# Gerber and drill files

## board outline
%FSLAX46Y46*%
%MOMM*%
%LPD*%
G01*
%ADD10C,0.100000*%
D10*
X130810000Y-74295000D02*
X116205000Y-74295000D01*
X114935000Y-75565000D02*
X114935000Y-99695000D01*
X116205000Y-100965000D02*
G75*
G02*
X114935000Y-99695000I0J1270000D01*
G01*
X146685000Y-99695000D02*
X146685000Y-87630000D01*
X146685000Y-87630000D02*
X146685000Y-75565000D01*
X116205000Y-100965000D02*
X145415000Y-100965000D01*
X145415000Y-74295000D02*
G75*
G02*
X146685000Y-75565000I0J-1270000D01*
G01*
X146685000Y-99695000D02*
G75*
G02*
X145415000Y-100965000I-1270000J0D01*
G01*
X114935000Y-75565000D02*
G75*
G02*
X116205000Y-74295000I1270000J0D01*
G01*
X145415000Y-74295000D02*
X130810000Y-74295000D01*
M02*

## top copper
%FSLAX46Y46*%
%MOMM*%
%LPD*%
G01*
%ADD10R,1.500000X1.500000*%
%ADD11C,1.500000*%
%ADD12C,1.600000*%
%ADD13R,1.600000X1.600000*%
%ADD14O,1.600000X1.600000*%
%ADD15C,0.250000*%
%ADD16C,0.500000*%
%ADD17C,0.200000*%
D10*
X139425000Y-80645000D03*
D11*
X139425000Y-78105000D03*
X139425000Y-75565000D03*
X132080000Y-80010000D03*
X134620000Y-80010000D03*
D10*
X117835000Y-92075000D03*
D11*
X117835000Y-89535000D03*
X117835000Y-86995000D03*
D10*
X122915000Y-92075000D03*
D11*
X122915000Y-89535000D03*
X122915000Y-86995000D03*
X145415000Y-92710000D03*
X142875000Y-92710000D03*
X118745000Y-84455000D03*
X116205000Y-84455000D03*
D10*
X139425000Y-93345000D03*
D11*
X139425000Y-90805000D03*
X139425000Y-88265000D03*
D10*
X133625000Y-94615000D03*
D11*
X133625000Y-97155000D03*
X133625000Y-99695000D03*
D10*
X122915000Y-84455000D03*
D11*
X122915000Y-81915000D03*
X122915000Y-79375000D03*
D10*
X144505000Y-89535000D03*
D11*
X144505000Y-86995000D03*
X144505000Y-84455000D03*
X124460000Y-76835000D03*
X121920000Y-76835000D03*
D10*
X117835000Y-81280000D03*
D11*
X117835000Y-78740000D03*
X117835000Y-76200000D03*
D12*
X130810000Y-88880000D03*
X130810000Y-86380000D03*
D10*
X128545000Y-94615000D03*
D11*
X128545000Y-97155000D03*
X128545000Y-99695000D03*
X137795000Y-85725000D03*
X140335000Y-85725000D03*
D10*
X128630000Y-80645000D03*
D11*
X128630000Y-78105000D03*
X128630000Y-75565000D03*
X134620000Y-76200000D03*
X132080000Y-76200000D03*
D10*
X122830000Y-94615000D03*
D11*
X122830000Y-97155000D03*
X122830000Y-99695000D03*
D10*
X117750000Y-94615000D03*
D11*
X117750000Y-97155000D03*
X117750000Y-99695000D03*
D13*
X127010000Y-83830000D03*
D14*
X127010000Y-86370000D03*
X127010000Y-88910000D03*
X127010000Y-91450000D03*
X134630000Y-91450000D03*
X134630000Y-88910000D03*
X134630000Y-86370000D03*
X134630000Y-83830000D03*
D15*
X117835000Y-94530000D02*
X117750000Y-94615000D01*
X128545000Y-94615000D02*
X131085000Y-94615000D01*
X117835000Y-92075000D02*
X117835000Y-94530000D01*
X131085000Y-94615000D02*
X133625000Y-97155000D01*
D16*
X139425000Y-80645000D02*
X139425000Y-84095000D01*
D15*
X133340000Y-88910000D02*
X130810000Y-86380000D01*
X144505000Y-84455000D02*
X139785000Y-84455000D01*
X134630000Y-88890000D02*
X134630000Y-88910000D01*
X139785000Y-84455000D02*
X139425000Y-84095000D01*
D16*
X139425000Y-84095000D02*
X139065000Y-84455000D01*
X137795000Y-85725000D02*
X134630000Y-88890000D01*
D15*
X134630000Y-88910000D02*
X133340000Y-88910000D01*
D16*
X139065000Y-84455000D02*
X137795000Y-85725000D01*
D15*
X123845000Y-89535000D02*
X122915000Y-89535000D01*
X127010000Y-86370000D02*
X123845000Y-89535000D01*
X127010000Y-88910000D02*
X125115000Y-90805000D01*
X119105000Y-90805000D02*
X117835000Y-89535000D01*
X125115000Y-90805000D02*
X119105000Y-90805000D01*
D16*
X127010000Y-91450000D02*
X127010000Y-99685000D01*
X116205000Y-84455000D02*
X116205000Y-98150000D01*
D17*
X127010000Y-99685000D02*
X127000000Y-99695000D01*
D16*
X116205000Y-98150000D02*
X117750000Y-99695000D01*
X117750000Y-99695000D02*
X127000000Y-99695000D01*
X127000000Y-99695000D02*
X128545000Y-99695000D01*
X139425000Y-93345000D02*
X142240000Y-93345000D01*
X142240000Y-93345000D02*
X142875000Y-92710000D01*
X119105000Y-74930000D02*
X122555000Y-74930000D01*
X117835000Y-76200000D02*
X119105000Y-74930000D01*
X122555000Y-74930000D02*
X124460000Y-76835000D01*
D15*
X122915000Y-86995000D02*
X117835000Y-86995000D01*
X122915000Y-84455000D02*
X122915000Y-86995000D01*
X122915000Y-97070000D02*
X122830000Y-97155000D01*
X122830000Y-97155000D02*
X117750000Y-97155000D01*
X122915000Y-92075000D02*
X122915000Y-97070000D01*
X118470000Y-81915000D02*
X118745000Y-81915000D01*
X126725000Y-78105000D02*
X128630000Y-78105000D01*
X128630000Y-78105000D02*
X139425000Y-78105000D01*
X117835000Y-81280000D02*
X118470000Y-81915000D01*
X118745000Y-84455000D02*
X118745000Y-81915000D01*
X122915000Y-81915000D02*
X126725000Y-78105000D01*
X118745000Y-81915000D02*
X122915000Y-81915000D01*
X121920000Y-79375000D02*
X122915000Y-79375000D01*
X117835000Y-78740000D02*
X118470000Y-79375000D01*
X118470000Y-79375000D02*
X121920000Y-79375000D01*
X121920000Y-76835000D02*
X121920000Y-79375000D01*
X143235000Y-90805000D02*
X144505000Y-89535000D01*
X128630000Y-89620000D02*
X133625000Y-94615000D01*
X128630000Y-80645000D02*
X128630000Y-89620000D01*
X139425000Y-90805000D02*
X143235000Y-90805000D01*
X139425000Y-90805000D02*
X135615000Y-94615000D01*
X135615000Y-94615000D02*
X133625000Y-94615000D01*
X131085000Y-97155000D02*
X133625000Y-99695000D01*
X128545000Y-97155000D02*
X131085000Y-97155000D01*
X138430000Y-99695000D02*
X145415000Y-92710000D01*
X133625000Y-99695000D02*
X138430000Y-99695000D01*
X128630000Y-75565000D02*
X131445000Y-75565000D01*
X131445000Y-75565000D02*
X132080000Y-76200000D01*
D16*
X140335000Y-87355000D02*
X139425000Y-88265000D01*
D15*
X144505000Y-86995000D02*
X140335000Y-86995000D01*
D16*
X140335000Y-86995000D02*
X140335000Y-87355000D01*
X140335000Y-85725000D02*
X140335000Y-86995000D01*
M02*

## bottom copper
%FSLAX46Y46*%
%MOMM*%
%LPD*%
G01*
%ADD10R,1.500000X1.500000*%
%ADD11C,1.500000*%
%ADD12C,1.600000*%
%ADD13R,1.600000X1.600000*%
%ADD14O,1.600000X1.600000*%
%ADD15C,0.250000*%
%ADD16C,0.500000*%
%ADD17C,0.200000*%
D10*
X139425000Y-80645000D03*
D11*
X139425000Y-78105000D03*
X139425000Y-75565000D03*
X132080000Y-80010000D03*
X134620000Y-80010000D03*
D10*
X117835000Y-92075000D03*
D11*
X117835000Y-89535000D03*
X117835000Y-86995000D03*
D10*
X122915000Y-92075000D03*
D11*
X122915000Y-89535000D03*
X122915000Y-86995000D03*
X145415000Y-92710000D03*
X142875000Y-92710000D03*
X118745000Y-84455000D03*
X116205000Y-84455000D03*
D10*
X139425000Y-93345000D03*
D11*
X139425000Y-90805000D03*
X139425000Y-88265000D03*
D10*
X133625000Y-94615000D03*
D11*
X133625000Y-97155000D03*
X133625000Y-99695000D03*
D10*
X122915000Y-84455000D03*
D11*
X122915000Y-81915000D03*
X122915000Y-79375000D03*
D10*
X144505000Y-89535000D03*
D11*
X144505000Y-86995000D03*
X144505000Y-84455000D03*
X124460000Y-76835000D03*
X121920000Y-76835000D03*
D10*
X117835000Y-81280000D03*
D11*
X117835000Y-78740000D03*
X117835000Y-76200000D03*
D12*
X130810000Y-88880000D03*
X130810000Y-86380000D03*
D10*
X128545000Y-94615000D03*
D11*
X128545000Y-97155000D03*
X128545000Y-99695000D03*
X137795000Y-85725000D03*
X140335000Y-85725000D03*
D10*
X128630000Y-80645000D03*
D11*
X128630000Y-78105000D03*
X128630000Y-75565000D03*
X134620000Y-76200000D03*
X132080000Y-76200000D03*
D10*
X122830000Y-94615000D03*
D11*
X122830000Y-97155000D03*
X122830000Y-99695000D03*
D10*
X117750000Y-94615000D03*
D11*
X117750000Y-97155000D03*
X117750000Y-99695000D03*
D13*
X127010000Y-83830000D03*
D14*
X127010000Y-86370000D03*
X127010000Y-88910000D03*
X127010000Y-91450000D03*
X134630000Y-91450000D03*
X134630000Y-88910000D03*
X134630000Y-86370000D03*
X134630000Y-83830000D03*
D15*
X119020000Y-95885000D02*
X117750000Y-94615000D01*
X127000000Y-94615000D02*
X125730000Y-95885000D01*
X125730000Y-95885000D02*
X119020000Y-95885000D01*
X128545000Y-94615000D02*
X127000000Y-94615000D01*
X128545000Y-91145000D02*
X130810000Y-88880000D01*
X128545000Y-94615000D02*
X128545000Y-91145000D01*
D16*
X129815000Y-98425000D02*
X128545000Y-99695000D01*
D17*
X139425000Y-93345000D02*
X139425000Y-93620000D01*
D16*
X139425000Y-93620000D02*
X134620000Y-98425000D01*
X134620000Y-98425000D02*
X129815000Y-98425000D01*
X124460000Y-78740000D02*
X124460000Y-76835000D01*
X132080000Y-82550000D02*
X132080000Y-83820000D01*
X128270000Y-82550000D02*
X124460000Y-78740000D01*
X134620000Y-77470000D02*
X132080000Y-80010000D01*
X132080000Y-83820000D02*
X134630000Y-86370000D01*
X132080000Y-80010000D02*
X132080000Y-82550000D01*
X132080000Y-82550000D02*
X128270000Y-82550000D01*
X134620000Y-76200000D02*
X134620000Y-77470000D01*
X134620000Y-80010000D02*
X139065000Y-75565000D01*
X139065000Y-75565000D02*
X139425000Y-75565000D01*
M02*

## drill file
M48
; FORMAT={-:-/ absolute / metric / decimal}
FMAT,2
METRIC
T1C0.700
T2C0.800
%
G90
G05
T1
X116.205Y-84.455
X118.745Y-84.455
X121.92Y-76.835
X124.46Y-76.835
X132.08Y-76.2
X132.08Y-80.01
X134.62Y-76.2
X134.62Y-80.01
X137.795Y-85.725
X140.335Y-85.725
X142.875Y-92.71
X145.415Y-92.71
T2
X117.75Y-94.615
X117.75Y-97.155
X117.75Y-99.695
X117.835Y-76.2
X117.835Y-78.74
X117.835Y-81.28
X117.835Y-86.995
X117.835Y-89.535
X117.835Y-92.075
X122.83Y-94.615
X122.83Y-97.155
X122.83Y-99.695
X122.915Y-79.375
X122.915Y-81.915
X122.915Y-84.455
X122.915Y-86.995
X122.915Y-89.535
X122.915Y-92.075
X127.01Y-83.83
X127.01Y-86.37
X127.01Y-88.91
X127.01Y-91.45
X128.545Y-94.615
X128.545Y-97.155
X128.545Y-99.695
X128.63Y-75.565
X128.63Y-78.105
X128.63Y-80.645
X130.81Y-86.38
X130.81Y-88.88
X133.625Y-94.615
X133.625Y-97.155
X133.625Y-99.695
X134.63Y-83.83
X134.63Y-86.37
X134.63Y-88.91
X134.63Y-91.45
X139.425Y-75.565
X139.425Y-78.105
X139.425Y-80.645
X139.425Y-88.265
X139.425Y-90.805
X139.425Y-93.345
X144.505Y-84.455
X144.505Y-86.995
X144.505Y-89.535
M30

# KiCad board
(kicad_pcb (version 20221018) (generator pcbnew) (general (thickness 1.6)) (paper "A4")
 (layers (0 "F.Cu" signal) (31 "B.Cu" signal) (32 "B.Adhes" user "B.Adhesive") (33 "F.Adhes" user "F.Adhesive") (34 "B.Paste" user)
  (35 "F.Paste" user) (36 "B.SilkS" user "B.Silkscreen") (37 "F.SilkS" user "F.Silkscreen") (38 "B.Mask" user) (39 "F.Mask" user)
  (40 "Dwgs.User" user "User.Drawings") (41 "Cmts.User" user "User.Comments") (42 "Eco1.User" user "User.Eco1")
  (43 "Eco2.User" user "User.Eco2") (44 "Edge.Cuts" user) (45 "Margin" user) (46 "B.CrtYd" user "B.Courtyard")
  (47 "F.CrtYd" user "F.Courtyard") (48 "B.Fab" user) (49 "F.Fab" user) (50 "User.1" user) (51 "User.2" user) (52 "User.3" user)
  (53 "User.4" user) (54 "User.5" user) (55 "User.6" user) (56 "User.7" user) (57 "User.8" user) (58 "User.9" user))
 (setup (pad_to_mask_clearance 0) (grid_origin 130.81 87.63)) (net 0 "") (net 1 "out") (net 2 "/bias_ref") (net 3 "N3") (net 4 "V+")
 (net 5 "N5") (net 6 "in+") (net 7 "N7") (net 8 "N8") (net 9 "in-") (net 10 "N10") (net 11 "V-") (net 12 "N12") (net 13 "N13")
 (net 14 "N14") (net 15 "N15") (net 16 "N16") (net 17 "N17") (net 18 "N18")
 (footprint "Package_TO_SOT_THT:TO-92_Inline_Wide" (layer "F.Cu") (at 139.425 80.645 90)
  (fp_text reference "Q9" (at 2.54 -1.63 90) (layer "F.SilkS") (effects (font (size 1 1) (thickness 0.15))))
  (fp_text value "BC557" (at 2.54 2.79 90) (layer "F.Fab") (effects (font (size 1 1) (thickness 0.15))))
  (pad "1" thru_hole rect (at 0 0 90) (size 1.5 1.5) (drill 0.8) (layers "*.Cu" "*.Mask") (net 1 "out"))
  (pad "2" thru_hole circle (at 2.54 0 90) (size 1.5 1.5) (drill 0.8) (layers "*.Cu" "*.Mask") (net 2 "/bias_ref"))
  (pad "3" thru_hole circle (at 5.08 0 90) (size 1.5 1.5) (drill 0.8) (layers "*.Cu" "*.Mask") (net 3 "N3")))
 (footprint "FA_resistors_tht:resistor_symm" (layer "F.Cu") (at 133.35 80.01)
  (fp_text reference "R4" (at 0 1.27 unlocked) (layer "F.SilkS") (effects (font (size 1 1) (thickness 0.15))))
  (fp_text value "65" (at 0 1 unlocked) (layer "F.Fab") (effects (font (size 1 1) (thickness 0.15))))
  (pad "1" thru_hole circle (at -1.27 0) (size 1.5 1.5) (drill 0.7) (layers "*.Cu" "*.Mask") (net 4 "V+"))
  (pad "2" thru_hole circle (at 1.27 0) (size 1.5 1.5) (drill 0.7) (layers "*.Cu" "*.Mask") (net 3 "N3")))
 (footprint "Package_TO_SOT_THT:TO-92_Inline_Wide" (layer "F.Cu") (at 117.835 92.075 90)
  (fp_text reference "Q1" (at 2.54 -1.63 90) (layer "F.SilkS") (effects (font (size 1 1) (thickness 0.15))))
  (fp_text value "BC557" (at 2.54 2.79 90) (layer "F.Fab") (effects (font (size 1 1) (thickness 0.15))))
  (pad "1" thru_hole rect (at 0 0 90) (size 1.5 1.5) (drill 0.8) (layers "*.Cu" "*.Mask") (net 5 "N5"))
  (pad "2" thru_hole circle (at 2.54 0 90) (size 1.5 1.5) (drill 0.8) (layers "*.Cu" "*.Mask") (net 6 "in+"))
  (pad "3" thru_hole circle (at 5.08 0 90) (size 1.5 1.5) (drill 0.8) (layers "*.Cu" "*.Mask") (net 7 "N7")))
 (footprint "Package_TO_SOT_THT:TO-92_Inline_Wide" (layer "F.Cu") (at 122.915 92.075 90)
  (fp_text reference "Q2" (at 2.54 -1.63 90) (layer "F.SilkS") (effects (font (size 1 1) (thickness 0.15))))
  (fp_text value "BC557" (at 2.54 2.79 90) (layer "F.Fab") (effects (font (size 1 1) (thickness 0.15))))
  (pad "1" thru_hole rect (at 0 0 90) (size 1.5 1.5) (drill 0.8) (layers "*.Cu" "*.Mask") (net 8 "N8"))
  (pad "2" thru_hole circle (at 2.54 0 90) (size 1.5 1.5) (drill 0.8) (layers "*.Cu" "*.Mask") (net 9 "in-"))
  (pad "3" thru_hole circle (at 5.08 0 90) (size 1.5 1.5) (drill 0.8) (layers "*.Cu" "*.Mask") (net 7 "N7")))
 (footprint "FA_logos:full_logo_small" (layer "F.Cu") (at 141.31 97.63 90)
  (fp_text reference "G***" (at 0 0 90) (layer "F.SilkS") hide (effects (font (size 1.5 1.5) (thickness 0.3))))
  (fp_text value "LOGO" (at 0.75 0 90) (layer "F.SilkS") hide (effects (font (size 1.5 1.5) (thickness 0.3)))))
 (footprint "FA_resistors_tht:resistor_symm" (layer "F.Cu") (at 144.145 92.71 180)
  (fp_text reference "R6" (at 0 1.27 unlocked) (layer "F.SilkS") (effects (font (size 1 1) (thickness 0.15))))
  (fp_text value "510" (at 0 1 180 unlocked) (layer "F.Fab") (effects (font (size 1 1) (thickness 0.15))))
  (pad "1" thru_hole circle (at -1.27 0 180) (size 1.5 1.5) (drill 0.7) (layers "*.Cu" "*.Mask") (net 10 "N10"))
  (pad "2" thru_hole circle (at 1.27 0 180) (size 1.5 1.5) (drill 0.7) (layers "*.Cu" "*.Mask") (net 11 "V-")))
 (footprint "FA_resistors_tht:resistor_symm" (layer "F.Cu") (at 117.475 84.455 180)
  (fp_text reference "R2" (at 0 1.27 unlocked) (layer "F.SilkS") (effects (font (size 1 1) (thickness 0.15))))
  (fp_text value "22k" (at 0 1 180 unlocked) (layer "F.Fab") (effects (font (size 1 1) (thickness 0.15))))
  (pad "1" thru_hole circle (at -1.27 0 180) (size 1.5 1.5) (drill 0.7) (layers "*.Cu" "*.Mask") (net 2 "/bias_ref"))
  (pad "2" thru_hole circle (at 1.27 0 180) (size 1.5 1.5) (drill 0.7) (layers "*.Cu" "*.Mask") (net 11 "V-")))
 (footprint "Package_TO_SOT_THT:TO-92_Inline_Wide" (layer "F.Cu") (at 139.425 93.345 90)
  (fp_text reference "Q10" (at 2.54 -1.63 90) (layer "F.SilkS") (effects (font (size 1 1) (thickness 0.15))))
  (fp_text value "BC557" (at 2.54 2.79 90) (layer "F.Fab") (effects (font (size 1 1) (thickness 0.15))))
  (pad "1" thru_hole rect (at 0 0 90) (size 1.5 1.5) (drill 0.8) (layers "*.Cu" "*.Mask") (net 11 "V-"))
  (pad "2" thru_hole circle (at 2.54 0 90) (size 1.5 1.5) (drill 0.8) (layers "*.Cu" "*.Mask") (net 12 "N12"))
  (pad "3" thru_hole circle (at 5.08 0 90) (size 1.5 1.5) (drill 0.8) (layers "*.Cu" "*.Mask") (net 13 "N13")))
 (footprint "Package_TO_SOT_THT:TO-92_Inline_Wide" (layer "F.Cu") (at 133.625 94.615 -90)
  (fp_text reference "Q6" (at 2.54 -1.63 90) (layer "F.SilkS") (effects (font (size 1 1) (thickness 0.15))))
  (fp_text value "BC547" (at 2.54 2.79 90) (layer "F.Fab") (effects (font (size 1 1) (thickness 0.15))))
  (pad "1" thru_hole rect (at 0 0 270) (size 1.5 1.5) (drill 0.8) (layers "*.Cu" "*.Mask") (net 12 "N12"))
  (pad "2" thru_hole circle (at 2.54 0 270) (size 1.5 1.5) (drill 0.8) (layers "*.Cu" "*.Mask") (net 5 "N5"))
  (pad "3" thru_hole circle (at 5.08 0 270) (size 1.5 1.5) (drill 0.8) (layers "*.Cu" "*.Mask") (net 10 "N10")))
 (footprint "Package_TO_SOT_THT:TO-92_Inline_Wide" (layer "F.Cu") (at 122.915 84.455 90)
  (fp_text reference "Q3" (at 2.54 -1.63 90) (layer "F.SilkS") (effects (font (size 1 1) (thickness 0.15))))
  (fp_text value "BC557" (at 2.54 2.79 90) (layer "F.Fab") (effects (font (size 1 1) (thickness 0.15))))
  (pad "1" thru_hole rect (at 0 0 90) (size 1.5 1.5) (drill 0.8) (layers "*.Cu" "*.Mask") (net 7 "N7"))
  (pad "2" thru_hole circle (at 2.54 0 90) (size 1.5 1.5) (drill 0.8) (layers "*.Cu" "*.Mask") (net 2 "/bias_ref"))
  (pad "3" thru_hole circle (at 5.08 0 90) (size 1.5 1.5) (drill 0.8) (layers "*.Cu" "*.Mask") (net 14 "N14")))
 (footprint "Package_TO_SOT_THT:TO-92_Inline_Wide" (layer "F.Cu") (at 144.505 89.535 90)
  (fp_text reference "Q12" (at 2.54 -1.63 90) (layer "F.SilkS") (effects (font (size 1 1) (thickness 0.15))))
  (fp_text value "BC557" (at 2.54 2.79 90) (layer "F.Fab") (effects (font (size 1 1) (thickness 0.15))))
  (pad "1" thru_hole rect (at 0 0 90) (size 1.5 1.5) (drill 0.8) (layers "*.Cu" "*.Mask") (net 12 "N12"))
  (pad "2" thru_hole circle (at 2.54 0 90) (size 1.5 1.5) (drill 0.8) (layers "*.Cu" "*.Mask") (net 13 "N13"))
  (pad "3" thru_hole circle (at 5.08 0 90) (size 1.5 1.5) (drill 0.8) (layers "*.Cu" "*.Mask") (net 1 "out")))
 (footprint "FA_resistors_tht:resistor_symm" (layer "F.Cu") (at 123.19 76.835 180)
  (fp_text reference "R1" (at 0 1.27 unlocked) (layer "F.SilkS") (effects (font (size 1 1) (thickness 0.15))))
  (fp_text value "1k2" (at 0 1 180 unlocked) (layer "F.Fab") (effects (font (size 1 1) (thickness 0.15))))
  (pad "1" thru_hole circle (at -1.27 0 180) (size 1.5 1.5) (drill 0.7) (layers "*.Cu" "*.Mask") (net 4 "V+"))
  (pad "2" thru_hole circle (at 1.27 0 180) (size 1.5 1.5) (drill 0.7) (layers "*.Cu" "*.Mask") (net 14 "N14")))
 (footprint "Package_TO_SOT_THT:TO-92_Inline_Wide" (layer "F.Cu") (at 117.835 81.28 90)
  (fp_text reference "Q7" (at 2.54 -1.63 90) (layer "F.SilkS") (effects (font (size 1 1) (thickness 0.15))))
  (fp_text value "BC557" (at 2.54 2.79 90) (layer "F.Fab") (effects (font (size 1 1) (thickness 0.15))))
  (pad "1" thru_hole rect (at 0 0 90) (size 1.5 1.5) (drill 0.8) (layers "*.Cu" "*.Mask") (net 2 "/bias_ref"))
  (pad "2" thru_hole circle (at 2.54 0 90) (size 1.5 1.5) (drill 0.8) (layers "*.Cu" "*.Mask") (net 14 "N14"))
  (pad "3" thru_hole circle (at 5.08 0 90) (size 1.5 1.5) (drill 0.8) (layers "*.Cu" "*.Mask") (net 4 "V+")))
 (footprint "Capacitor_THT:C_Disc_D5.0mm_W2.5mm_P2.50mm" (layer "F.Cu") (at 130.81 88.88 90)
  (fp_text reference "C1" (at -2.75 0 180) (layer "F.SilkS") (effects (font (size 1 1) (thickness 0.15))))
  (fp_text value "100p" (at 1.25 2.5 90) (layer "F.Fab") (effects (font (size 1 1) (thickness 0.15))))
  (pad "1" thru_hole circle (at 0 0 90) (size 1.6 1.6) (drill 0.8) (layers "*.Cu" "*.Mask") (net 5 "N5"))
  (pad "2" thru_hole circle (at 2.5 0 90) (size 1.6 1.6) (drill 0.8) (layers "*.Cu" "*.Mask") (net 1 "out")))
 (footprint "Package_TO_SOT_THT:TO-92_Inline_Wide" (layer "F.Cu") (at 128.545 94.615 -90)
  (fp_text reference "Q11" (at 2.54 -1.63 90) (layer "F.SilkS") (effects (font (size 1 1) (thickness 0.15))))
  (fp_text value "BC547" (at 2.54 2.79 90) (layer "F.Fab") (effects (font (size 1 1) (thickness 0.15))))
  (pad "1" thru_hole rect (at 0 0 270) (size 1.5 1.5) (drill 0.8) (layers "*.Cu" "*.Mask") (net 5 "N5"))
  (pad "2" thru_hole circle (at 2.54 0 270) (size 1.5 1.5) (drill 0.8) (layers "*.Cu" "*.Mask") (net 10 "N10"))
  (pad "3" thru_hole circle (at 5.08 0 270) (size 1.5 1.5) (drill 0.8) (layers "*.Cu" "*.Mask") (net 11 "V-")))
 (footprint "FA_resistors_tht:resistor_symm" (layer "F.Cu") (at 139.065 85.725)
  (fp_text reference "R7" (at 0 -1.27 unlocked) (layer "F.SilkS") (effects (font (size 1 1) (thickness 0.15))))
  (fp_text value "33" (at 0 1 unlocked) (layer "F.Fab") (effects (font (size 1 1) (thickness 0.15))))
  (pad "1" thru_hole circle (at -1.27 0) (size 1.5 1.5) (drill 0.7) (layers "*.Cu" "*.Mask") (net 1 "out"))
  (pad "2" thru_hole circle (at 1.27 0) (size 1.5 1.5) (drill 0.7) (layers "*.Cu" "*.Mask") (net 13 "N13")))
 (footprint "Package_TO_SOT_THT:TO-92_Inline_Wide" (layer "F.Cu") (at 128.63 80.645 90)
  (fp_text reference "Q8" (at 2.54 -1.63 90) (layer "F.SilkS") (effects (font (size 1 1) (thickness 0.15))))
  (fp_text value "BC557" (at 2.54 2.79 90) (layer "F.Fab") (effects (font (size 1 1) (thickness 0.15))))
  (pad "1" thru_hole rect (at 0 0 90) (size 1.5 1.5) (drill 0.8) (layers "*.Cu" "*.Mask") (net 12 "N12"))
  (pad "2" thru_hole circle (at 2.54 0 90) (size 1.5 1.5) (drill 0.8) (layers "*.Cu" "*.Mask") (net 2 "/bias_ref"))
  (pad "3" thru_hole circle (at 5.08 0 90) (size 1.5 1.5) (drill 0.8) (layers "*.Cu" "*.Mask") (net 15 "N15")))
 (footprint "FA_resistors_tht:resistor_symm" (layer "F.Cu") (at 133.35 76.2 180)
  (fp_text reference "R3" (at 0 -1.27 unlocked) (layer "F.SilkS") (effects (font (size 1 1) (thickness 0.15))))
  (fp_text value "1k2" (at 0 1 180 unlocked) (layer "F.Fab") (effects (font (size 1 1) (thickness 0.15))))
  (pad "1" thru_hole circle (at -1.27 0 180) (size 1.5 1.5) (drill 0.7) (layers "*.Cu" "*.Mask") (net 4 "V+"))
  (pad "2" thru_hole circle (at 1.27 0 180) (size 1.5 1.5) (drill 0.7) (layers "*.Cu" "*.Mask") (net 15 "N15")))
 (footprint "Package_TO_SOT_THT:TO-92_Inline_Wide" (layer "F.Cu") (at 122.83 94.615 -90)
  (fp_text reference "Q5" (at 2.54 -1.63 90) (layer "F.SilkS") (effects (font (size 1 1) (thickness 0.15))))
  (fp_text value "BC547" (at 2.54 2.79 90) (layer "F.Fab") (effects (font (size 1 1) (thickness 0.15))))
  (pad "1" thru_hole rect (at 0 0 270) (size 1.5 1.5) (drill 0.8) (layers "*.Cu" "*.Mask") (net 8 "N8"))
  (pad "2" thru_hole circle (at 2.54 0 270) (size 1.5 1.5) (drill 0.8) (layers "*.Cu" "*.Mask") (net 8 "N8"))
  (pad "3" thru_hole circle (at 5.08 0 270) (size 1.5 1.5) (drill 0.8) (layers "*.Cu" "*.Mask") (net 11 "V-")))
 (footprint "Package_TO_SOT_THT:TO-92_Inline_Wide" (layer "F.Cu") (at 117.75 94.615 -90)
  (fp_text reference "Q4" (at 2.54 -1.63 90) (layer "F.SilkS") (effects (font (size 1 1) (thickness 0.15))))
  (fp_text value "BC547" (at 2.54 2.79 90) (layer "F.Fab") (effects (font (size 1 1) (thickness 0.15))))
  (pad "1" thru_hole rect (at 0 0 270) (size 1.5 1.5) (drill 0.8) (layers "*.Cu" "*.Mask") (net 5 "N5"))
  (pad "2" thru_hole circle (at 2.54 0 270) (size 1.5 1.5) (drill 0.8) (layers "*.Cu" "*.Mask") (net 8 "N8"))
  (pad "3" thru_hole circle (at 5.08 0 270) (size 1.5 1.5) (drill 0.8) (layers "*.Cu" "*.Mask") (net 11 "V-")))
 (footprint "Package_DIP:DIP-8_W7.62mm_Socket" (layer "F.Cu") (at 127.01 83.83)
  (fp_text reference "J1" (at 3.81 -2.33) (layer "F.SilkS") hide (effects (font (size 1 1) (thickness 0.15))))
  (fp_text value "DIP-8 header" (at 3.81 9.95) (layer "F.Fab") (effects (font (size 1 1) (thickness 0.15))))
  (pad "1" thru_hole rect (at 0 0) (size 1.6 1.6) (drill 0.8) (layers "*.Cu" "*.Mask") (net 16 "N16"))
  (pad "2" thru_hole oval (at 0 2.54) (size 1.6 1.6) (drill 0.8) (layers "*.Cu" "*.Mask") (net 9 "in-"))
  (pad "3" thru_hole oval (at 0 5.08) (size 1.6 1.6) (drill 0.8) (layers "*.Cu" "*.Mask") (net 6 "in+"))
  (pad "4" thru_hole oval (at 0 7.62) (size 1.6 1.6) (drill 0.8) (layers "*.Cu" "*.Mask") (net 11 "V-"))
  (pad "5" thru_hole oval (at 7.62 7.62) (size 1.6 1.6) (drill 0.8) (layers "*.Cu" "*.Mask") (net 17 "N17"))
  (pad "6" thru_hole oval (at 7.62 5.08) (size 1.6 1.6) (drill 0.8) (layers "*.Cu" "*.Mask") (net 1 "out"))
  (pad "7" thru_hole oval (at 7.62 2.54) (size 1.6 1.6) (drill 0.8) (layers "*.Cu" "*.Mask") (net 4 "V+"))
  (pad "8" thru_hole oval (at 7.62 0) (size 1.6 1.6) (drill 0.8) (layers "*.Cu" "*.Mask") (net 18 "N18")))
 (gr_line (start 130.81 74.295) (end 116.205 74.295) (stroke (width 0.1) (type default)) (layer "Edge.Cuts"))
 (gr_line (start 114.935 75.565) (end 114.935 99.695) (stroke (width 0.1) (type default)) (layer "Edge.Cuts"))
 (gr_arc (start 116.205 100.965) (mid 115.306974 100.593026) (end 114.935 99.695) (stroke (width 0.1) (type default)) (layer "Edge.Cuts"))
 (gr_line (start 146.685 99.695) (end 146.685 87.63) (stroke (width 0.1) (type default)) (layer "Edge.Cuts"))
 (gr_line (start 146.685 87.63) (end 146.685 75.565) (stroke (width 0.1) (type default)) (layer "Edge.Cuts"))
 (gr_line (start 116.205 100.965) (end 145.415 100.965) (stroke (width 0.1) (type default)) (layer "Edge.Cuts"))
 (gr_arc (start 145.415 74.295) (mid 146.313026 74.666974) (end 146.685 75.565) (stroke (width 0.1) (type default)) (layer "Edge.Cuts"))
 (gr_arc (start 146.685 99.695) (mid 146.313026 100.593026) (end 145.415 100.965) (stroke (width 0.1) (type default)) (layer "Edge.Cuts"))
 (gr_arc (start 114.935 75.565) (mid 115.306974 74.666974) (end 116.205 74.295) (stroke (width 0.1) (type default)) (layer "Edge.Cuts"))
 (gr_line (start 145.415 74.295) (end 130.81 74.295) (stroke (width 0.1) (type default)) (layer "Edge.Cuts"))
 (segment (start 117.835 94.53) (end 117.75 94.615) (width 0.25) (layer "F.Cu") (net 5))
 (segment (start 128.545 94.615) (end 131.085 94.615) (width 0.25) (layer "F.Cu") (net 5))
 (segment (start 117.835 92.075) (end 117.835 94.53) (width 0.25) (layer "F.Cu") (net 5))
 (segment (start 131.085 94.615) (end 133.625 97.155) (width 0.25) (layer "F.Cu") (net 5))
 (segment (start 119.02 95.885) (end 117.75 94.615) (width 0.25) (layer "B.Cu") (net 5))
 (segment (start 127 94.615) (end 125.73 95.885) (width 0.25) (layer "B.Cu") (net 5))
 (segment (start 125.73 95.885) (end 119.02 95.885) (width 0.25) (layer "B.Cu") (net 5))
 (segment (start 128.545 94.615) (end 127 94.615) (width 0.25) (layer "B.Cu") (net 5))
 (segment (start 128.545 91.145) (end 130.81 88.88) (width 0.25) (layer "B.Cu") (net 5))
 (segment (start 128.545 94.615) (end 128.545 91.145) (width 0.25) (layer "B.Cu") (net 5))
 (segment (start 139.425 80.645) (end 139.425 84.095) (width 0.5) (layer "F.Cu") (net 1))
 (segment (start 133.34 88.91) (end 130.81 86.38) (width 0.25) (layer "F.Cu") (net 1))
 (segment (start 144.505 84.455) (end 139.785 84.455) (width 0.25) (layer "F.Cu") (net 1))
 (segment (start 134.63 88.89) (end 134.63 88.91) (width 0.25) (layer "F.Cu") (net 1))
 (segment (start 139.785 84.455) (end 139.425 84.095) (width 0.25) (layer "F.Cu") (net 1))
 (segment (start 139.425 84.095) (end 139.065 84.455) (width 0.5) (layer "F.Cu") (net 1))
 (segment (start 137.795 85.725) (end 134.63 88.89) (width 0.5) (layer "F.Cu") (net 1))
 (segment (start 134.63 88.91) (end 133.34 88.91) (width 0.25) (layer "F.Cu") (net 1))
 (segment (start 139.065 84.455) (end 137.795 85.725) (width 0.5) (layer "F.Cu") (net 1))
 (segment (start 123.845 89.535) (end 122.915 89.535) (width 0.25) (layer "F.Cu") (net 9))
 (segment (start 127.01 86.37) (end 123.845 89.535) (width 0.25) (layer "F.Cu") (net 9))
 (segment (start 127.01 88.91) (end 125.115 90.805) (width 0.25) (layer "F.Cu") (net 6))
 (segment (start 119.105 90.805) (end 117.835 89.535) (width 0.25) (layer "F.Cu") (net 6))
 (segment (start 125.115 90.805) (end 119.105 90.805) (width 0.25) (layer "F.Cu") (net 6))
 (segment (start 127.01 91.45) (end 127.01 99.685) (width 0.5) (layer "F.Cu") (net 11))
 (segment (start 116.205 84.455) (end 116.205 98.15) (width 0.5) (layer "F.Cu") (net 11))
 (segment (start 127.01 99.685) (end 127 99.695) (width 0.2) (layer "F.Cu") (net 11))
 (segment (start 116.205 98.15) (end 117.75 99.695) (width 0.5) (layer "F.Cu") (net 11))
 (segment (start 117.75 99.695) (end 127 99.695) (width 0.5) (layer "F.Cu") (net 11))
 (segment (start 127 99.695) (end 128.545 99.695) (width 0.5) (layer "F.Cu") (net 11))
 (segment (start 139.425 93.345) (end 142.24 93.345) (width 0.5) (layer "F.Cu") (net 11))
 (segment (start 142.24 93.345) (end 142.875 92.71) (width 0.5) (layer "F.Cu") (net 11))
 (segment (start 129.815 98.425) (end 128.545 99.695) (width 0.5) (layer "B.Cu") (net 11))
 (segment (start 139.425 93.345) (end 139.425 93.62) (width 0.2) (layer "B.Cu") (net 11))
 (segment (start 139.425 93.62) (end 134.62 98.425) (width 0.5) (layer "B.Cu") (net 11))
 (segment (start 134.62 98.425) (end 129.815 98.425) (width 0.5) (layer "B.Cu") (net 11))
 (segment (start 119.105 74.93) (end 122.555 74.93) (width 0.5) (layer "F.Cu") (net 4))
 (segment (start 117.835 76.2) (end 119.105 74.93) (width 0.5) (layer "F.Cu") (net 4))
 (segment (start 122.555 74.93) (end 124.46 76.835) (width 0.5) (layer "F.Cu") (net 4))
 (segment (start 124.46 78.74) (end 124.46 76.835) (width 0.5) (layer "B.Cu") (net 4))
 (segment (start 132.08 82.55) (end 132.08 83.82) (width 0.5) (layer "B.Cu") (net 4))
 (segment (start 128.27 82.55) (end 124.46 78.74) (width 0.5) (layer "B.Cu") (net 4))
 (segment (start 134.62 77.47) (end 132.08 80.01) (width 0.5) (layer "B.Cu") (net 4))
 (segment (start 132.08 83.82) (end 134.63 86.37) (width 0.5) (layer "B.Cu") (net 4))
 (segment (start 132.08 80.01) (end 132.08 82.55) (width 0.5) (layer "B.Cu") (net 4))
 (segment (start 132.08 82.55) (end 128.27 82.55) (width 0.5) (layer "B.Cu") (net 4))
 (segment (start 134.62 76.2) (end 134.62 77.47) (width 0.5) (layer "B.Cu") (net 4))
 (segment (start 122.915 86.995) (end 117.835 86.995) (width 0.25) (layer "F.Cu") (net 7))
 (segment (start 122.915 84.455) (end 122.915 86.995) (width 0.25) (layer "F.Cu") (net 7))
 (segment (start 122.915 97.07) (end 122.83 97.155) (width 0.25) (layer "F.Cu") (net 8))
 (segment (start 122.83 97.155) (end 117.75 97.155) (width 0.25) (layer "F.Cu") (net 8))
 (segment (start 122.915 92.075) (end 122.915 97.07) (width 0.25) (layer "F.Cu") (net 8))
 (segment (start 118.47 81.915) (end 118.745 81.915) (width 0.25) (layer "F.Cu") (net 2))
 (segment (start 126.725 78.105) (end 128.63 78.105) (width 0.25) (layer "F.Cu") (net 2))
 (segment (start 128.63 78.105) (end 139.425 78.105) (width 0.25) (layer "F.Cu") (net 2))
 (segment (start 117.835 81.28) (end 118.47 81.915) (width 0.25) (layer "F.Cu") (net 2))
 (segment (start 118.745 84.455) (end 118.745 81.915) (width 0.25) (layer "F.Cu") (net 2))
 (segment (start 122.915 81.915) (end 126.725 78.105) (width 0.25) (layer "F.Cu") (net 2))
 (segment (start 118.745 81.915) (end 122.915 81.915) (width 0.25) (layer "F.Cu") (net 2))
 (segment (start 121.92 79.375) (end 122.915 79.375) (width 0.25) (layer "F.Cu") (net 14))
 (segment (start 117.835 78.74) (end 118.47 79.375) (width 0.25) (layer "F.Cu") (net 14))
 (segment (start 118.47 79.375) (end 121.92 79.375) (width 0.25) (layer "F.Cu") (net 14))
 (segment (start 121.92 76.835) (end 121.92 79.375) (width 0.25) (layer "F.Cu") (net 14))
 (segment (start 143.235 90.805) (end 144.505 89.535) (width 0.25) (layer "F.Cu") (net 12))
 (segment (start 128.63 89.62) (end 133.625 94.615) (width 0.25) (layer "F.Cu") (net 12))
 (segment (start 128.63 80.645) (end 128.63 89.62) (width 0.25) (layer "F.Cu") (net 12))
 (segment (start 139.425 90.805) (end 143.235 90.805) (width 0.25) (layer "F.Cu") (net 12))
 (segment (start 139.425 90.805) (end 135.615 94.615) (width 0.25) (layer "F.Cu") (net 12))
 (segment (start 135.615 94.615) (end 133.625 94.615) (width 0.25) (layer "F.Cu") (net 12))
 (segment (start 131.085 97.155) (end 133.625 99.695) (width 0.25) (layer "F.Cu") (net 10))
 (segment (start 128.545 97.155) (end 131.085 97.155) (width 0.25) (layer "F.Cu") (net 10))
 (segment (start 138.43 99.695) (end 145.415 92.71) (width 0.25) (layer "F.Cu") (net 10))
 (segment (start 133.625 99.695) (end 138.43 99.695) (width 0.25) (layer "F.Cu") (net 10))
 (segment (start 128.63 75.565) (end 131.445 75.565) (width 0.25) (layer "F.Cu") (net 15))
 (segment (start 131.445 75.565) (end 132.08 76.2) (width 0.25) (layer "F.Cu") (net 15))
 (segment (start 134.62 80.01) (end 139.065 75.565) (width 0.5) (layer "B.Cu") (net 3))
 (segment (start 139.065 75.565) (end 139.425 75.565) (width 0.5) (layer "B.Cu") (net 3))
 (segment (start 140.335 87.355) (end 139.425 88.265) (width 0.5) (layer "F.Cu") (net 13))
 (segment (start 144.505 86.995) (end 140.335 86.995) (width 0.25) (layer "F.Cu") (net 13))
 (segment (start 140.335 86.995) (end 140.335 87.355) (width 0.5) (layer "F.Cu") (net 13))
 (segment (start 140.335 85.725) (end 140.335 86.995) (width 0.5) (layer "F.Cu") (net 13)))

